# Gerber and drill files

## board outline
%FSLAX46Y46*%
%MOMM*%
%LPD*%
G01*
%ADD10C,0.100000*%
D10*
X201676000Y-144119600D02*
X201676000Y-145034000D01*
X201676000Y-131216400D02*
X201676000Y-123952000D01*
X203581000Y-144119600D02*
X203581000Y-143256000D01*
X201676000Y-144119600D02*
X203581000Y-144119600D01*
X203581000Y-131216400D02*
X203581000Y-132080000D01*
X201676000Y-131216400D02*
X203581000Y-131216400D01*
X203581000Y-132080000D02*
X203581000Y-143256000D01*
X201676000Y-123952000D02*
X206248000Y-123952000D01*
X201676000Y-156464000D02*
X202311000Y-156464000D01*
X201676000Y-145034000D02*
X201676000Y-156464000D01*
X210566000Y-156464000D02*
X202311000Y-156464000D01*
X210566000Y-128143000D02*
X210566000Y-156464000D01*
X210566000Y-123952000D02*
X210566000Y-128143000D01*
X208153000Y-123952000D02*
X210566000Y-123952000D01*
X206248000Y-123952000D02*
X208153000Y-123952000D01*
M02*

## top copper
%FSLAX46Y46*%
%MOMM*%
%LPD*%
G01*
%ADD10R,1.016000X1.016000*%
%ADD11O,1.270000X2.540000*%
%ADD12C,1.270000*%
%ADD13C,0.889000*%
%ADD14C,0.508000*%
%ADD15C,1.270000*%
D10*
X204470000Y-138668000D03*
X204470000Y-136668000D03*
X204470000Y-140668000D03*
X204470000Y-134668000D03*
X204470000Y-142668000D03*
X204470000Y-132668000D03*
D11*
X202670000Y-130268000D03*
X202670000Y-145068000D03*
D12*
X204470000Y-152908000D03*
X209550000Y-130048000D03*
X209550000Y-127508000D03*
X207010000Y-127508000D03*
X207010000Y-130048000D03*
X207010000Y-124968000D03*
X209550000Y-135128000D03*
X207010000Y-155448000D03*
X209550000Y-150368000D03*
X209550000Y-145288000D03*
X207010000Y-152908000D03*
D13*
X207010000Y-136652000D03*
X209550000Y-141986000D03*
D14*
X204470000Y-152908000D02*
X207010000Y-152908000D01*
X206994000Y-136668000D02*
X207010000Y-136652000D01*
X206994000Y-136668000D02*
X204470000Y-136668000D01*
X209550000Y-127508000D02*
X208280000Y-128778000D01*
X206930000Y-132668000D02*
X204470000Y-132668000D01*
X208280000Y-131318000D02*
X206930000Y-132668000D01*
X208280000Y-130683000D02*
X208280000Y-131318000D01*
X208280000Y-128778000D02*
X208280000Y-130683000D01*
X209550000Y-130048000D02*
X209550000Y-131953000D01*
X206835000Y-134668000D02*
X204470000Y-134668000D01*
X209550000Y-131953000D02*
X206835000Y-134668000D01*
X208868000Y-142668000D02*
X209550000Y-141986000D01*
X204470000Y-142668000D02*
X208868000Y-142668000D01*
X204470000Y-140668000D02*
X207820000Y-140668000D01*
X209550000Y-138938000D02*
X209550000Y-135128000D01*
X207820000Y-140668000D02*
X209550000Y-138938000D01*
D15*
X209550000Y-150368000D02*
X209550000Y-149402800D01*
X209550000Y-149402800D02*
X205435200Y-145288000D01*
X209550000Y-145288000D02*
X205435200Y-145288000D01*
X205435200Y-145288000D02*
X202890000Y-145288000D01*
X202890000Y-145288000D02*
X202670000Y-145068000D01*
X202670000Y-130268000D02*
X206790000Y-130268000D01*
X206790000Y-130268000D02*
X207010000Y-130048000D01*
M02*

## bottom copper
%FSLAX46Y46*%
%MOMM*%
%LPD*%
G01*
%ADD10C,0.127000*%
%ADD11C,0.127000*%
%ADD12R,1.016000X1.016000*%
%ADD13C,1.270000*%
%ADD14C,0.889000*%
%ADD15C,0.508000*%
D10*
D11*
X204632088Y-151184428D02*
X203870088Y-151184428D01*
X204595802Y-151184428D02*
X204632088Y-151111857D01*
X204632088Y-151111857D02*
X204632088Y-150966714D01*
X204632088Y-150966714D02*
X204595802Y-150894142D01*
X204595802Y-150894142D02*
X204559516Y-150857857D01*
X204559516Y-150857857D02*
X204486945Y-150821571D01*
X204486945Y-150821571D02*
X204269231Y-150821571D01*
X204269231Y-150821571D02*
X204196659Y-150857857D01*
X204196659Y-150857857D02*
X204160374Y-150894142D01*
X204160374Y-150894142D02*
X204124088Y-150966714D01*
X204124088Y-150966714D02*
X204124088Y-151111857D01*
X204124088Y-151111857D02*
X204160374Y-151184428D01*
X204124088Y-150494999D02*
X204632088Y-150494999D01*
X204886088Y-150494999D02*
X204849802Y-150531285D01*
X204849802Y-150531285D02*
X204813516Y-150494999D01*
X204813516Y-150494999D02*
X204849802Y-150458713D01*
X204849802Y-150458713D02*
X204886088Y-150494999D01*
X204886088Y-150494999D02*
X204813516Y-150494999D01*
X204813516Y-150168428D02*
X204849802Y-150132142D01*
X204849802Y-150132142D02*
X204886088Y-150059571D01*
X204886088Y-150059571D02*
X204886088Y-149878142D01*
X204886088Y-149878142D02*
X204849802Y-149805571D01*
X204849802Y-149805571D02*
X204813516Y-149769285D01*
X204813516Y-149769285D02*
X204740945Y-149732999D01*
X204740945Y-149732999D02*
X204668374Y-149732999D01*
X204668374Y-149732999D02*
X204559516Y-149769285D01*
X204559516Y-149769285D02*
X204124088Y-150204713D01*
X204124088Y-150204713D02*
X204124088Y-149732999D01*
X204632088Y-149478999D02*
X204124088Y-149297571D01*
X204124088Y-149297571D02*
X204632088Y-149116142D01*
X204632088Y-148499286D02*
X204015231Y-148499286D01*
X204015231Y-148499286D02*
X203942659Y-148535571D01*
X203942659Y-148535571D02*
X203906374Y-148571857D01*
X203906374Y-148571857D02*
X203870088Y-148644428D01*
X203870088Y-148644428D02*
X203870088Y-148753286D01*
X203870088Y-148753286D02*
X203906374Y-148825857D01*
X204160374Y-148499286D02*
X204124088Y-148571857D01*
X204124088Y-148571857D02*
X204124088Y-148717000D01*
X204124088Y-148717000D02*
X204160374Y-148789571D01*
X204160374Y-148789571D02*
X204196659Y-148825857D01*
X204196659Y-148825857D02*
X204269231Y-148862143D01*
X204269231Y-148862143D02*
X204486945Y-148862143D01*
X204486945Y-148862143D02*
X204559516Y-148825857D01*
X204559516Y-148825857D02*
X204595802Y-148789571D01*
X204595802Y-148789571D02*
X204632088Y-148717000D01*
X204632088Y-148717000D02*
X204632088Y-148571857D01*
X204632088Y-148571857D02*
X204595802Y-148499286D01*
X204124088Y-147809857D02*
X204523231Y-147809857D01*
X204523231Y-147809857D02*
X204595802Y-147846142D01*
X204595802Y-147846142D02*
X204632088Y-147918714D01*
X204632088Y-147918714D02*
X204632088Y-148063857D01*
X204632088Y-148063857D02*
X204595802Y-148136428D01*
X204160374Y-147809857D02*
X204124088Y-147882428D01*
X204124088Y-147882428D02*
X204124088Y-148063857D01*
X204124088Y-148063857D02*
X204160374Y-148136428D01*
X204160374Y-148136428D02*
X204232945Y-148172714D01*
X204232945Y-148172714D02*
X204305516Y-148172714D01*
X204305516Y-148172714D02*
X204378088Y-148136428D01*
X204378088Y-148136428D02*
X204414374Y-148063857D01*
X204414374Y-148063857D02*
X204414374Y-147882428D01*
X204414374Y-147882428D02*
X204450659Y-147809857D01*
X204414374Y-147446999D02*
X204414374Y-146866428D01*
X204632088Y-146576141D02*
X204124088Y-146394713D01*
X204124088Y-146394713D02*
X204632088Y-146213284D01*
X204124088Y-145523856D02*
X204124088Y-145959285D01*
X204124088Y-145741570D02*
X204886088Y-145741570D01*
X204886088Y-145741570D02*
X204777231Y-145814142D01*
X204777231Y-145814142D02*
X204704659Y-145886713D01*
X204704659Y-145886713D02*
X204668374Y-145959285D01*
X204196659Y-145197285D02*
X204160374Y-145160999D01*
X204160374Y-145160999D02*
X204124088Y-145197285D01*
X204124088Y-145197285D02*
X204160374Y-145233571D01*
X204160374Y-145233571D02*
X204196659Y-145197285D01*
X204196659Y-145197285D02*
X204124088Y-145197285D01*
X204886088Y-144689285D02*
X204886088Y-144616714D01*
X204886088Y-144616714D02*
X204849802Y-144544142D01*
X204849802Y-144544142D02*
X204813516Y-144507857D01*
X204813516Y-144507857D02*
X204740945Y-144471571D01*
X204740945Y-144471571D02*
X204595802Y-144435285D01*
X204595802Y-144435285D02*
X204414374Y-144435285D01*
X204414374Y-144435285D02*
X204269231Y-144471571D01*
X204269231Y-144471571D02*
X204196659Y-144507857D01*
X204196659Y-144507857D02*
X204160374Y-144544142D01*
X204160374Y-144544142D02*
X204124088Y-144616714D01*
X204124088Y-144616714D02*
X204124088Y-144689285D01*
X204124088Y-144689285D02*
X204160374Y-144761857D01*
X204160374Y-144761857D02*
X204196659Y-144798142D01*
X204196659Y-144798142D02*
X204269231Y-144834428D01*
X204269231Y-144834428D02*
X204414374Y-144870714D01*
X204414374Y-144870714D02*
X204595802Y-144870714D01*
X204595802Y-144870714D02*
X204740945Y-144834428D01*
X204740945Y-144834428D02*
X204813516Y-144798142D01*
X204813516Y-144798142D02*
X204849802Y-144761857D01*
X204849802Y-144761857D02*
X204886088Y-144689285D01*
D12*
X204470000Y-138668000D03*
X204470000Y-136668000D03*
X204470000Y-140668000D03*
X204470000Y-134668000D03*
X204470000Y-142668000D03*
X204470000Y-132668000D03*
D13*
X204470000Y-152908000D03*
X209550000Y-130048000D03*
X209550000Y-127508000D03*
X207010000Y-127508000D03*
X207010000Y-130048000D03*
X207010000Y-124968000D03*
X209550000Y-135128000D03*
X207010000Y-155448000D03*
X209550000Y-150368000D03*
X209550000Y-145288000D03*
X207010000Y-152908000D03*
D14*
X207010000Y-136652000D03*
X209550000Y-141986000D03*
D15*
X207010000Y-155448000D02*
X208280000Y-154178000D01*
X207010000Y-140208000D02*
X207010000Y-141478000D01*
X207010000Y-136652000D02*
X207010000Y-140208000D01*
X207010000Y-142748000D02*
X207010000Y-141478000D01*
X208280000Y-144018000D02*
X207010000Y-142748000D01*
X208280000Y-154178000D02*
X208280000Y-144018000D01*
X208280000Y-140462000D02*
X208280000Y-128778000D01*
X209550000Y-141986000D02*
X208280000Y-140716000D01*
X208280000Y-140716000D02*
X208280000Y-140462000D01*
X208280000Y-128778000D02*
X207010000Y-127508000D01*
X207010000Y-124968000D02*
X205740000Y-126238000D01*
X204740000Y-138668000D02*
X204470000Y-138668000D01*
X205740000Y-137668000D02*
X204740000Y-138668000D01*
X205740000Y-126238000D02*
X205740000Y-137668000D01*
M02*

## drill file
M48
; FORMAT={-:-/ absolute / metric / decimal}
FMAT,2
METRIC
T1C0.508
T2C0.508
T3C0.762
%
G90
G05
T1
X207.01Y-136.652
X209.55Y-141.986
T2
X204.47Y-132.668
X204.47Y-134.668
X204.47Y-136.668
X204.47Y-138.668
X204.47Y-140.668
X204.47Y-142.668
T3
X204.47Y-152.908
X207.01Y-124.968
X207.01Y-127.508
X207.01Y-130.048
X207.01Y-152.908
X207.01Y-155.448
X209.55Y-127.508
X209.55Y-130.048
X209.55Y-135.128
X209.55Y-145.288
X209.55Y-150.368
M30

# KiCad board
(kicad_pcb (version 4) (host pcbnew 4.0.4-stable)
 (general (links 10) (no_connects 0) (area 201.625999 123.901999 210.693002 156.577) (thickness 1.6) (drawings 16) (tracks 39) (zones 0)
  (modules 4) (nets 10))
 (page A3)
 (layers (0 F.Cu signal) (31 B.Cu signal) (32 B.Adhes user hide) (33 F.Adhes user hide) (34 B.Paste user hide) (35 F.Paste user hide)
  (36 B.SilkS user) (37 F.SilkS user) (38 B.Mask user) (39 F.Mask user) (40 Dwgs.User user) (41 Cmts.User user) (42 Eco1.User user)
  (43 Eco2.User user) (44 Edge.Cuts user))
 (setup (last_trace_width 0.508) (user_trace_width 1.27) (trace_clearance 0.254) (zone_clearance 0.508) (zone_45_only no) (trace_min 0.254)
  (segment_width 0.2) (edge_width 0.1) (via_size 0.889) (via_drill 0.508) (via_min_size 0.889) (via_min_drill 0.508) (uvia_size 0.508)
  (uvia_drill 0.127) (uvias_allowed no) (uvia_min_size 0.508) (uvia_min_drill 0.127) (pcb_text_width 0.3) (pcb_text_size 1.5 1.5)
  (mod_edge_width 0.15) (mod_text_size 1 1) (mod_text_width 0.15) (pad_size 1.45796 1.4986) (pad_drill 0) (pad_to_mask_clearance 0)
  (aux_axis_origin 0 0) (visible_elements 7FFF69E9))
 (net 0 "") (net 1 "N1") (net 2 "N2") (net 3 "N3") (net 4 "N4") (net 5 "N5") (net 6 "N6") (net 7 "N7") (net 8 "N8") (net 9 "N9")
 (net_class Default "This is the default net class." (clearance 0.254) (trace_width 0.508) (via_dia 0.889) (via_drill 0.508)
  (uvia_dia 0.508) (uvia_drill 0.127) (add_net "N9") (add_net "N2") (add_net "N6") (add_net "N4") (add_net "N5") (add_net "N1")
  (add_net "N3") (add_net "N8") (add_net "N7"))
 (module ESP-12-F (layer F.Cu) (at 204.47 137.668)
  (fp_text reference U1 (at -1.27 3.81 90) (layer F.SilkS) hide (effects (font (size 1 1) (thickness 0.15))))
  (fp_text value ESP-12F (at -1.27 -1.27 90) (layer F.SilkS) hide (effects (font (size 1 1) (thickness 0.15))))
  (pad 12 thru_hole rect (at 0 1) (size 1.016 1.016) (drill 0.508) (layers *.Cu *.Mask) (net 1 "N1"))
  (pad 11 thru_hole rect (at 0 -1) (size 1.016 1.016) (drill 0.508) (layers *.Cu *.Mask) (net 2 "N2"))
  (pad 13 thru_hole rect (at 0 3) (size 1.016 1.016) (drill 0.508) (layers *.Cu *.Mask) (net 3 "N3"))
  (pad 10 thru_hole rect (at 0 -3) (size 1.016 1.016) (drill 0.508) (layers *.Cu *.Mask) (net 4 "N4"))
  (pad 14 thru_hole rect (at 0 5) (size 1.016 1.016) (drill 0.508) (layers *.Cu *.Mask) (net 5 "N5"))
  (pad 9 thru_hole rect (at 0 -5) (size 1.016 1.016) (drill 0.508) (layers *.Cu *.Mask) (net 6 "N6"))
  (pad 8 smd oval (at -1.8 -7.4) (size 1.27 2.54) (layers F.Cu F.Paste F.Mask) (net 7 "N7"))
  (pad 15 smd oval (at -1.8 7.4) (size 1.27 2.54) (layers F.Cu F.Paste F.Mask) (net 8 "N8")))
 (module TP (layer F.Cu) (at 204.47 152.908)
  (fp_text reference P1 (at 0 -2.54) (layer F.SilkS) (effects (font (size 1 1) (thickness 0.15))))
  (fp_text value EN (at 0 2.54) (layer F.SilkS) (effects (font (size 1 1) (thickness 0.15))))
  (pad 1 thru_hole circle (at 0 0) (size 1.27 1.27) (drill 0.762) (layers *.Cu *.Mask) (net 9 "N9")))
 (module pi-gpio (layer F.Cu) (at 207.01 130.048)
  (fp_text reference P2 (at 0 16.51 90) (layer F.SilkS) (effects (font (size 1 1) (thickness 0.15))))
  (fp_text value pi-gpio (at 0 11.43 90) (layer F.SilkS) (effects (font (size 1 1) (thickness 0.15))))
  (pad 18 thru_hole circle (at 2.54 0) (size 1.27 1.27) (drill 0.762) (layers *.Cu *.Mask) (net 4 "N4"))
  (pad 16 thru_hole circle (at 2.54 -2.54) (size 1.27 1.27) (drill 0.762) (layers *.Cu *.Mask) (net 6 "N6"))
  (pad 15 thru_hole circle (at 0 -2.54) (size 1.27 1.27) (drill 0.762) (layers *.Cu *.Mask) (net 5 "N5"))
  (pad 17 thru_hole circle (at 0 0) (size 1.27 1.27) (drill 0.762) (layers *.Cu *.Mask) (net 7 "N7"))
  (pad 13 thru_hole circle (at 0 -5.08) (size 1.27 1.27) (drill 0.762) (layers *.Cu *.Mask) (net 1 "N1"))
  (pad 22 thru_hole circle (at 2.54 5.08) (size 1.27 1.27) (drill 0.762) (layers *.Cu *.Mask) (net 3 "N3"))
  (pad 37 thru_hole circle (at 0 25.4) (size 1.27 1.27) (drill 0.762) (layers *.Cu *.Mask) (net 2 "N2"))
  (pad 34 thru_hole circle (at 2.54 20.32) (size 1.27 1.27) (drill 0.762) (layers *.Cu *.Mask) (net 8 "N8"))
  (pad 30 thru_hole circle (at 2.54 15.24) (size 1.27 1.27) (drill 0.762) (layers *.Cu *.Mask) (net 8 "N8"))
  (pad 35 thru_hole circle (at 0 22.86) (size 1.27 1.27) (drill 0.762) (layers *.Cu *.Mask) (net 9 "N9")))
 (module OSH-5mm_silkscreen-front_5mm (layer F.Cu) (at 204.724 149.098 270)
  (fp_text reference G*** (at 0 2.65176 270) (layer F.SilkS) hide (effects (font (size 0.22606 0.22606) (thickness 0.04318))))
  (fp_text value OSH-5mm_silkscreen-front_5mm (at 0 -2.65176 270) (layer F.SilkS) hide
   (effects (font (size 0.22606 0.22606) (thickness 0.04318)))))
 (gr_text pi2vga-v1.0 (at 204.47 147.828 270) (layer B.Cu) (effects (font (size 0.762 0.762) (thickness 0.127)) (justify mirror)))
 (gr_line (start 201.676 144.1196) (end 201.676 145.034) (angle 90) (layer Edge.Cuts) (width 0.1))
 (gr_line (start 201.676 131.2164) (end 201.676 123.952) (angle 90) (layer Edge.Cuts) (width 0.1))
 (gr_line (start 203.581 144.1196) (end 203.581 143.256) (angle 90) (layer Edge.Cuts) (width 0.1))
 (gr_line (start 201.676 144.1196) (end 203.581 144.1196) (angle 90) (layer Edge.Cuts) (width 0.1))
 (gr_line (start 203.581 131.2164) (end 203.581 132.08) (angle 90) (layer Edge.Cuts) (width 0.1))
 (gr_line (start 201.676 131.2164) (end 203.581 131.2164) (angle 90) (layer Edge.Cuts) (width 0.1))
 (gr_line (start 203.581 132.08) (end 203.581 143.256) (angle 90) (layer Edge.Cuts) (width 0.1))
 (gr_line (start 201.676 123.952) (end 206.248 123.952) (angle 90) (layer Edge.Cuts) (width 0.1))
 (gr_line (start 201.676 156.464) (end 202.311 156.464) (angle 90) (layer Edge.Cuts) (width 0.1))
 (gr_line (start 201.676 145.034) (end 201.676 156.464) (angle 90) (layer Edge.Cuts) (width 0.1))
 (gr_line (start 210.566 156.464) (end 202.311 156.464) (angle 90) (layer Edge.Cuts) (width 0.1))
 (gr_line (start 210.566 128.143) (end 210.566 156.464) (angle 90) (layer Edge.Cuts) (width 0.1))
 (gr_line (start 210.566 123.952) (end 210.566 128.143) (angle 90) (layer Edge.Cuts) (width 0.1))
 (gr_line (start 208.153 123.952) (end 210.566 123.952) (angle 90) (layer Edge.Cuts) (width 0.1))
 (gr_line (start 206.248 123.952) (end 208.153 123.952) (angle 90) (layer Edge.Cuts) (width 0.1))
 (segment (start 204.47 152.908) (end 207.01 152.908) (width 0.508) (layer F.Cu) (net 9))
 (segment (start 207.01 155.448) (end 208.28 154.178) (width 0.508) (layer B.Cu) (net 2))
 (segment (start 207.01 140.208) (end 207.01 141.478) (width 0.508) (layer B.Cu) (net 2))
 (segment (start 207.01 136.652) (end 207.01 140.208) (width 0.508) (layer B.Cu) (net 2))
 (via (at 207.01 136.652) (size 0.889) (layers F.Cu B.Cu) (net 2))
 (segment (start 206.994 136.668) (end 207.01 136.652) (width 0.508) (layer F.Cu) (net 2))
 (segment (start 206.994 136.668) (end 204.47 136.668) (width 0.508) (layer F.Cu) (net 2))
 (segment (start 207.01 142.748) (end 207.01 141.478) (width 0.508) (layer B.Cu) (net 2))
 (segment (start 208.28 144.018) (end 207.01 142.748) (width 0.508) (layer B.Cu) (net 2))
 (segment (start 208.28 154.178) (end 208.28 144.018) (width 0.508) (layer B.Cu) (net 2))
 (segment (start 209.55 127.508) (end 208.28 128.778) (width 0.508) (layer F.Cu) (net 6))
 (segment (start 206.93 132.668) (end 204.47 132.668) (width 0.508) (layer F.Cu) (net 6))
 (segment (start 208.28 131.318) (end 206.93 132.668) (width 0.508) (layer F.Cu) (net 6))
 (segment (start 208.28 130.683) (end 208.28 131.318) (width 0.508) (layer F.Cu) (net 6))
 (segment (start 208.28 128.778) (end 208.28 130.683) (width 0.508) (layer F.Cu) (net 6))
 (segment (start 209.55 130.048) (end 209.55 131.953) (width 0.508) (layer F.Cu) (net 4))
 (segment (start 206.835 134.668) (end 204.47 134.668) (width 0.508) (layer F.Cu) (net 4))
 (segment (start 209.55 131.953) (end 206.835 134.668) (width 0.508) (layer F.Cu) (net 4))
 (segment (start 208.28 140.462) (end 208.28 128.778) (width 0.508) (layer B.Cu) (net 5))
 (segment (start 208.868 142.668) (end 209.55 141.986) (width 0.508) (layer F.Cu) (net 5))
 (via (at 209.55 141.986) (size 0.889) (layers F.Cu B.Cu) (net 5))
 (segment (start 209.55 141.986) (end 208.28 140.716) (width 0.508) (layer B.Cu) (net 5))
 (segment (start 208.28 140.716) (end 208.28 140.462) (width 0.508) (layer B.Cu) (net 5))
 (segment (start 204.47 142.668) (end 208.868 142.668) (width 0.508) (layer F.Cu) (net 5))
 (segment (start 208.28 128.778) (end 207.01 127.508) (width 0.508) (layer B.Cu) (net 5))
 (segment (start 207.01 124.968) (end 205.74 126.238) (width 0.508) (layer B.Cu) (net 1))
 (segment (start 204.74 138.668) (end 204.47 138.668) (width 0.508) (layer B.Cu) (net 1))
 (segment (start 205.74 137.668) (end 204.74 138.668) (width 0.508) (layer B.Cu) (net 1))
 (segment (start 205.74 126.238) (end 205.74 137.668) (width 0.508) (layer B.Cu) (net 1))
 (segment (start 204.47 140.668) (end 207.82 140.668) (width 0.508) (layer F.Cu) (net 3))
 (segment (start 209.55 138.938) (end 209.55 135.128) (width 0.508) (layer F.Cu) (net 3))
 (segment (start 207.82 140.668) (end 209.55 138.938) (width 0.508) (layer F.Cu) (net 3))
 (segment (start 209.55 150.368) (end 209.55 149.4028) (width 1.27) (layer F.Cu) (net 8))
 (segment (start 209.55 149.4028) (end 205.4352 145.288) (width 1.27) (layer F.Cu) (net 8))
 (segment (start 209.55 145.288) (end 205.4352 145.288) (width 1.27) (layer F.Cu) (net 8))
 (segment (start 205.4352 145.288) (end 202.89 145.288) (width 1.27) (layer F.Cu) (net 8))
 (segment (start 202.89 145.288) (end 202.67 145.068) (width 1.27) (layer F.Cu) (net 8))
 (segment (start 202.67 130.268) (end 206.79 130.268) (width 1.27) (layer F.Cu) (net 7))
 (segment (start 206.79 130.268) (end 207.01 130.048) (width 1.27) (layer F.Cu) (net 7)))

